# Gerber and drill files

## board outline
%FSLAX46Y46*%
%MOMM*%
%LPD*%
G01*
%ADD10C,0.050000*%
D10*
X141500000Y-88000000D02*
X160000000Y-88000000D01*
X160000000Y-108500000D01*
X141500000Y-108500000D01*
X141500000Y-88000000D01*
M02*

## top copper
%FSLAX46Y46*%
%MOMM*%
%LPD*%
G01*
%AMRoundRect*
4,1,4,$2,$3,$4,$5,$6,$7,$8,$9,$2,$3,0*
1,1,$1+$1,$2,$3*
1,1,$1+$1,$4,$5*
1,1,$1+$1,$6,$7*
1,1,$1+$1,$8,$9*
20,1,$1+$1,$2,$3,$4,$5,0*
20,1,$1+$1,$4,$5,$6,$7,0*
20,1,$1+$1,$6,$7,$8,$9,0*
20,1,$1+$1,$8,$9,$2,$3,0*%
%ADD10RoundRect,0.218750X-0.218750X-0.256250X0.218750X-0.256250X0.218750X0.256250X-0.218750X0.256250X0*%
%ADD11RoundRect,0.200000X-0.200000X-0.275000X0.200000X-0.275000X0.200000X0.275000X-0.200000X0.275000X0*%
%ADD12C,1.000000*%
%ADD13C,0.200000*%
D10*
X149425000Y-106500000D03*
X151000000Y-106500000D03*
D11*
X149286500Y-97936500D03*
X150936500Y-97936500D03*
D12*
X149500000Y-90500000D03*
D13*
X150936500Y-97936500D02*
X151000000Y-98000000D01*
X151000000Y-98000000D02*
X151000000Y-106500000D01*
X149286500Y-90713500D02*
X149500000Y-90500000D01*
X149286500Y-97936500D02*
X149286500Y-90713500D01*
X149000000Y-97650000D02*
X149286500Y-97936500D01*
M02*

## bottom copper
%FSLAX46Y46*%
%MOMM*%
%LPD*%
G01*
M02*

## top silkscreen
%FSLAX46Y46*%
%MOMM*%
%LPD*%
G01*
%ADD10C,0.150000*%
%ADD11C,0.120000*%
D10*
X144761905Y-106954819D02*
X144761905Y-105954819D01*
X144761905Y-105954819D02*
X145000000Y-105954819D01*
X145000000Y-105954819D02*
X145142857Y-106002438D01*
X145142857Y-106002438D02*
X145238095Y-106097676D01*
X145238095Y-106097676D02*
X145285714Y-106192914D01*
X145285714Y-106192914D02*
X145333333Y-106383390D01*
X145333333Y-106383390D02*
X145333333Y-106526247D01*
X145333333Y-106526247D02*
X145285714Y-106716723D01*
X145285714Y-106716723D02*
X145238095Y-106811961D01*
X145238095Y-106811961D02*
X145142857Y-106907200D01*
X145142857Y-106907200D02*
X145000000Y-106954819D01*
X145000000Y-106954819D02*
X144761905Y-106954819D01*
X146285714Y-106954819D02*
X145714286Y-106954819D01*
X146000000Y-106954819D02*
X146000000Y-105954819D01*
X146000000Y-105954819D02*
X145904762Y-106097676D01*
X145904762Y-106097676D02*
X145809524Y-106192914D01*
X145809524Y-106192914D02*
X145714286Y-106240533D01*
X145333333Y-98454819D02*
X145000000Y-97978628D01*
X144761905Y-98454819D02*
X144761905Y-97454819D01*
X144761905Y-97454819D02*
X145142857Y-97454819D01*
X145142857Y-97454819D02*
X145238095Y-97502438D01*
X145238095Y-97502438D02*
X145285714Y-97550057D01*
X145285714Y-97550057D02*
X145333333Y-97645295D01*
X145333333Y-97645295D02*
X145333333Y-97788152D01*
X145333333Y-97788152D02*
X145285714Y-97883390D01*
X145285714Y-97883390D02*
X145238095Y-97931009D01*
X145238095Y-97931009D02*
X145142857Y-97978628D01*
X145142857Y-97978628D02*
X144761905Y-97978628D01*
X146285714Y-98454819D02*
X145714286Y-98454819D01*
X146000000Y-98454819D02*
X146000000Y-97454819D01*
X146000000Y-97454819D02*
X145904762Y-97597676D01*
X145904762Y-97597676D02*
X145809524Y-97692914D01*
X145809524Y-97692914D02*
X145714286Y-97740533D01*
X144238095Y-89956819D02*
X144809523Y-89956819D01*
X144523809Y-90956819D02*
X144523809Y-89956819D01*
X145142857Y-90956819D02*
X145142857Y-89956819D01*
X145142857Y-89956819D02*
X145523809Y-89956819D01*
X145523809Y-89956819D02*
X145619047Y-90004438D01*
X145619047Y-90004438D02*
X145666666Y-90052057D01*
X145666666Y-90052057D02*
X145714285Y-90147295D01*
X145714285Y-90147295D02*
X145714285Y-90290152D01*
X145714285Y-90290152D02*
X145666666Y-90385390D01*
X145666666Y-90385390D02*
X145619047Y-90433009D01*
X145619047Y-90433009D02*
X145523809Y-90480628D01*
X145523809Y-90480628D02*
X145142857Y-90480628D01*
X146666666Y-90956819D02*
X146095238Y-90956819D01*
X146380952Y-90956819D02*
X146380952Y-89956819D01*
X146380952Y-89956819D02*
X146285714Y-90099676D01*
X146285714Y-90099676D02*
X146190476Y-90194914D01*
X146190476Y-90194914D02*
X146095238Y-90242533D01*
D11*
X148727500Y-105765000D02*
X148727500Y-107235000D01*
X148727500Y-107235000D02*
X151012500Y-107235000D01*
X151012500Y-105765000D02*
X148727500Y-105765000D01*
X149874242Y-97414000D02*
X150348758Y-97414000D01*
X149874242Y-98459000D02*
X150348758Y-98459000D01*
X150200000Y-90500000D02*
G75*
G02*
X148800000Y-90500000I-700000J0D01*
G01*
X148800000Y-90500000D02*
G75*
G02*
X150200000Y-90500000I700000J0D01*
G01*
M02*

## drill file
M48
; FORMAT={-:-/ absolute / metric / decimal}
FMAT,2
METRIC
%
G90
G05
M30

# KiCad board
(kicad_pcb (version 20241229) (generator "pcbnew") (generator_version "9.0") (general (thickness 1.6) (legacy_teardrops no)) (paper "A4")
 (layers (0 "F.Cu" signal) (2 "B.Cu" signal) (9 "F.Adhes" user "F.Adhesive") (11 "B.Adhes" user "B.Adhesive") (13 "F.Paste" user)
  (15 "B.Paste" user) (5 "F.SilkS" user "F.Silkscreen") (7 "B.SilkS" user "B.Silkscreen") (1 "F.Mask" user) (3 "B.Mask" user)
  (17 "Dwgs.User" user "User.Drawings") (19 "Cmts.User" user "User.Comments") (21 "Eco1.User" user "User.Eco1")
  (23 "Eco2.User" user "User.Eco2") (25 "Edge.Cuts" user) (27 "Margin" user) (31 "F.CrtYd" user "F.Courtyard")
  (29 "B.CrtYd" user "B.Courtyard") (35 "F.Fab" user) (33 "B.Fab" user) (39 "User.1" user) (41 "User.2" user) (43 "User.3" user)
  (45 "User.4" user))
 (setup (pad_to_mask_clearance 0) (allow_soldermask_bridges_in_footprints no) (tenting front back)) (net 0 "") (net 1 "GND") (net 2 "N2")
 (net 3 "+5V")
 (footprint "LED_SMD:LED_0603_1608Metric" (layer "F.Cu") (at 150.2125 106.5)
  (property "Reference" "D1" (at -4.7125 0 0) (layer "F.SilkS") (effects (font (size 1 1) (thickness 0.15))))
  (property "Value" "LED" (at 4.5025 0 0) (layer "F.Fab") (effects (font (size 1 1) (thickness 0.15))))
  (fp_line (start -1.485 -0.735) (end -1.485 0.735) (stroke (width 0.12) (type solid)) (layer "F.SilkS"))
  (fp_line (start -1.485 0.735) (end 0.8 0.735) (stroke (width 0.12) (type solid)) (layer "F.SilkS"))
  (fp_line (start 0.8 -0.735) (end -1.485 -0.735) (stroke (width 0.12) (type solid)) (layer "F.SilkS"))
  (pad "1" smd roundrect (at -0.7875 0) (size 0.875 0.95) (layers "F.Cu" "F.Mask" "F.Paste") (roundrect_rratio 0.25) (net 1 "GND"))
  (pad "2" smd roundrect (at 0.7875 0) (size 0.875 0.95) (layers "F.Cu" "F.Mask" "F.Paste") (roundrect_rratio 0.25) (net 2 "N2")))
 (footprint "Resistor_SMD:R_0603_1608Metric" (layer "F.Cu") (at 150.1115 97.9365)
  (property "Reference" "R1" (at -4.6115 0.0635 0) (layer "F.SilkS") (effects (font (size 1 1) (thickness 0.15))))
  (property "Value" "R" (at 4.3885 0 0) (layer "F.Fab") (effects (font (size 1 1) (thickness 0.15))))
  (fp_line (start -0.237258 -0.5225) (end 0.237258 -0.5225) (stroke (width 0.12) (type solid)) (layer "F.SilkS"))
  (fp_line (start -0.237258 0.5225) (end 0.237258 0.5225) (stroke (width 0.12) (type solid)) (layer "F.SilkS"))
  (pad "1" smd roundrect (at -0.825 0) (size 0.8 0.95) (layers "F.Cu" "F.Mask" "F.Paste") (roundrect_rratio 0.25) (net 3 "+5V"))
  (pad "2" smd roundrect (at 0.825 0) (size 0.8 0.95) (layers "F.Cu" "F.Mask" "F.Paste") (roundrect_rratio 0.25) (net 2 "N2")))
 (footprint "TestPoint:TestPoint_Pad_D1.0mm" (layer "F.Cu") (at 149.5 90.5)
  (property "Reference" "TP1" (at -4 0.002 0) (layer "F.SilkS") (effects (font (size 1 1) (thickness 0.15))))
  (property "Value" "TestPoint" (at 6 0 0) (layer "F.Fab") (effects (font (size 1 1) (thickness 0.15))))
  (fp_circle (center 0 0) (end 0 0.7) (stroke (width 0.12) (type solid)) (fill no) (layer "F.SilkS"))
  (pad "1" smd circle (at 0 0) (size 1 1) (layers "F.Cu" "F.Mask") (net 3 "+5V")))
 (gr_rect (start 141.5 88) (end 160 108.5) (stroke (width 0.05) (type default)) (fill no) (layer "Edge.Cuts"))
 (segment (start 150.9365 97.9365) (end 151 98) (width 0.2) (layer "F.Cu") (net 2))
 (segment (start 151 98) (end 151 106.5) (width 0.2) (layer "F.Cu") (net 2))
 (segment (start 149.2865 90.7135) (end 149.5 90.5) (width 0.2) (layer "F.Cu") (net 3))
 (segment (start 149.2865 97.9365) (end 149.2865 90.7135) (width 0.2) (layer "F.Cu") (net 3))
 (segment (start 149 97.65) (end 149.2865 97.9365) (width 0.2) (layer "F.Cu") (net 3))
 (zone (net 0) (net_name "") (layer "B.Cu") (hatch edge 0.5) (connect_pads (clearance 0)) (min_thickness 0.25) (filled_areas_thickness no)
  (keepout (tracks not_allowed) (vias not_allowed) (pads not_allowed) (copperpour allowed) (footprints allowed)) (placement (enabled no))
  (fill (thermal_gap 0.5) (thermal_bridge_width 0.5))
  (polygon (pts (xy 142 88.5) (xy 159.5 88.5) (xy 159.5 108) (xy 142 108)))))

